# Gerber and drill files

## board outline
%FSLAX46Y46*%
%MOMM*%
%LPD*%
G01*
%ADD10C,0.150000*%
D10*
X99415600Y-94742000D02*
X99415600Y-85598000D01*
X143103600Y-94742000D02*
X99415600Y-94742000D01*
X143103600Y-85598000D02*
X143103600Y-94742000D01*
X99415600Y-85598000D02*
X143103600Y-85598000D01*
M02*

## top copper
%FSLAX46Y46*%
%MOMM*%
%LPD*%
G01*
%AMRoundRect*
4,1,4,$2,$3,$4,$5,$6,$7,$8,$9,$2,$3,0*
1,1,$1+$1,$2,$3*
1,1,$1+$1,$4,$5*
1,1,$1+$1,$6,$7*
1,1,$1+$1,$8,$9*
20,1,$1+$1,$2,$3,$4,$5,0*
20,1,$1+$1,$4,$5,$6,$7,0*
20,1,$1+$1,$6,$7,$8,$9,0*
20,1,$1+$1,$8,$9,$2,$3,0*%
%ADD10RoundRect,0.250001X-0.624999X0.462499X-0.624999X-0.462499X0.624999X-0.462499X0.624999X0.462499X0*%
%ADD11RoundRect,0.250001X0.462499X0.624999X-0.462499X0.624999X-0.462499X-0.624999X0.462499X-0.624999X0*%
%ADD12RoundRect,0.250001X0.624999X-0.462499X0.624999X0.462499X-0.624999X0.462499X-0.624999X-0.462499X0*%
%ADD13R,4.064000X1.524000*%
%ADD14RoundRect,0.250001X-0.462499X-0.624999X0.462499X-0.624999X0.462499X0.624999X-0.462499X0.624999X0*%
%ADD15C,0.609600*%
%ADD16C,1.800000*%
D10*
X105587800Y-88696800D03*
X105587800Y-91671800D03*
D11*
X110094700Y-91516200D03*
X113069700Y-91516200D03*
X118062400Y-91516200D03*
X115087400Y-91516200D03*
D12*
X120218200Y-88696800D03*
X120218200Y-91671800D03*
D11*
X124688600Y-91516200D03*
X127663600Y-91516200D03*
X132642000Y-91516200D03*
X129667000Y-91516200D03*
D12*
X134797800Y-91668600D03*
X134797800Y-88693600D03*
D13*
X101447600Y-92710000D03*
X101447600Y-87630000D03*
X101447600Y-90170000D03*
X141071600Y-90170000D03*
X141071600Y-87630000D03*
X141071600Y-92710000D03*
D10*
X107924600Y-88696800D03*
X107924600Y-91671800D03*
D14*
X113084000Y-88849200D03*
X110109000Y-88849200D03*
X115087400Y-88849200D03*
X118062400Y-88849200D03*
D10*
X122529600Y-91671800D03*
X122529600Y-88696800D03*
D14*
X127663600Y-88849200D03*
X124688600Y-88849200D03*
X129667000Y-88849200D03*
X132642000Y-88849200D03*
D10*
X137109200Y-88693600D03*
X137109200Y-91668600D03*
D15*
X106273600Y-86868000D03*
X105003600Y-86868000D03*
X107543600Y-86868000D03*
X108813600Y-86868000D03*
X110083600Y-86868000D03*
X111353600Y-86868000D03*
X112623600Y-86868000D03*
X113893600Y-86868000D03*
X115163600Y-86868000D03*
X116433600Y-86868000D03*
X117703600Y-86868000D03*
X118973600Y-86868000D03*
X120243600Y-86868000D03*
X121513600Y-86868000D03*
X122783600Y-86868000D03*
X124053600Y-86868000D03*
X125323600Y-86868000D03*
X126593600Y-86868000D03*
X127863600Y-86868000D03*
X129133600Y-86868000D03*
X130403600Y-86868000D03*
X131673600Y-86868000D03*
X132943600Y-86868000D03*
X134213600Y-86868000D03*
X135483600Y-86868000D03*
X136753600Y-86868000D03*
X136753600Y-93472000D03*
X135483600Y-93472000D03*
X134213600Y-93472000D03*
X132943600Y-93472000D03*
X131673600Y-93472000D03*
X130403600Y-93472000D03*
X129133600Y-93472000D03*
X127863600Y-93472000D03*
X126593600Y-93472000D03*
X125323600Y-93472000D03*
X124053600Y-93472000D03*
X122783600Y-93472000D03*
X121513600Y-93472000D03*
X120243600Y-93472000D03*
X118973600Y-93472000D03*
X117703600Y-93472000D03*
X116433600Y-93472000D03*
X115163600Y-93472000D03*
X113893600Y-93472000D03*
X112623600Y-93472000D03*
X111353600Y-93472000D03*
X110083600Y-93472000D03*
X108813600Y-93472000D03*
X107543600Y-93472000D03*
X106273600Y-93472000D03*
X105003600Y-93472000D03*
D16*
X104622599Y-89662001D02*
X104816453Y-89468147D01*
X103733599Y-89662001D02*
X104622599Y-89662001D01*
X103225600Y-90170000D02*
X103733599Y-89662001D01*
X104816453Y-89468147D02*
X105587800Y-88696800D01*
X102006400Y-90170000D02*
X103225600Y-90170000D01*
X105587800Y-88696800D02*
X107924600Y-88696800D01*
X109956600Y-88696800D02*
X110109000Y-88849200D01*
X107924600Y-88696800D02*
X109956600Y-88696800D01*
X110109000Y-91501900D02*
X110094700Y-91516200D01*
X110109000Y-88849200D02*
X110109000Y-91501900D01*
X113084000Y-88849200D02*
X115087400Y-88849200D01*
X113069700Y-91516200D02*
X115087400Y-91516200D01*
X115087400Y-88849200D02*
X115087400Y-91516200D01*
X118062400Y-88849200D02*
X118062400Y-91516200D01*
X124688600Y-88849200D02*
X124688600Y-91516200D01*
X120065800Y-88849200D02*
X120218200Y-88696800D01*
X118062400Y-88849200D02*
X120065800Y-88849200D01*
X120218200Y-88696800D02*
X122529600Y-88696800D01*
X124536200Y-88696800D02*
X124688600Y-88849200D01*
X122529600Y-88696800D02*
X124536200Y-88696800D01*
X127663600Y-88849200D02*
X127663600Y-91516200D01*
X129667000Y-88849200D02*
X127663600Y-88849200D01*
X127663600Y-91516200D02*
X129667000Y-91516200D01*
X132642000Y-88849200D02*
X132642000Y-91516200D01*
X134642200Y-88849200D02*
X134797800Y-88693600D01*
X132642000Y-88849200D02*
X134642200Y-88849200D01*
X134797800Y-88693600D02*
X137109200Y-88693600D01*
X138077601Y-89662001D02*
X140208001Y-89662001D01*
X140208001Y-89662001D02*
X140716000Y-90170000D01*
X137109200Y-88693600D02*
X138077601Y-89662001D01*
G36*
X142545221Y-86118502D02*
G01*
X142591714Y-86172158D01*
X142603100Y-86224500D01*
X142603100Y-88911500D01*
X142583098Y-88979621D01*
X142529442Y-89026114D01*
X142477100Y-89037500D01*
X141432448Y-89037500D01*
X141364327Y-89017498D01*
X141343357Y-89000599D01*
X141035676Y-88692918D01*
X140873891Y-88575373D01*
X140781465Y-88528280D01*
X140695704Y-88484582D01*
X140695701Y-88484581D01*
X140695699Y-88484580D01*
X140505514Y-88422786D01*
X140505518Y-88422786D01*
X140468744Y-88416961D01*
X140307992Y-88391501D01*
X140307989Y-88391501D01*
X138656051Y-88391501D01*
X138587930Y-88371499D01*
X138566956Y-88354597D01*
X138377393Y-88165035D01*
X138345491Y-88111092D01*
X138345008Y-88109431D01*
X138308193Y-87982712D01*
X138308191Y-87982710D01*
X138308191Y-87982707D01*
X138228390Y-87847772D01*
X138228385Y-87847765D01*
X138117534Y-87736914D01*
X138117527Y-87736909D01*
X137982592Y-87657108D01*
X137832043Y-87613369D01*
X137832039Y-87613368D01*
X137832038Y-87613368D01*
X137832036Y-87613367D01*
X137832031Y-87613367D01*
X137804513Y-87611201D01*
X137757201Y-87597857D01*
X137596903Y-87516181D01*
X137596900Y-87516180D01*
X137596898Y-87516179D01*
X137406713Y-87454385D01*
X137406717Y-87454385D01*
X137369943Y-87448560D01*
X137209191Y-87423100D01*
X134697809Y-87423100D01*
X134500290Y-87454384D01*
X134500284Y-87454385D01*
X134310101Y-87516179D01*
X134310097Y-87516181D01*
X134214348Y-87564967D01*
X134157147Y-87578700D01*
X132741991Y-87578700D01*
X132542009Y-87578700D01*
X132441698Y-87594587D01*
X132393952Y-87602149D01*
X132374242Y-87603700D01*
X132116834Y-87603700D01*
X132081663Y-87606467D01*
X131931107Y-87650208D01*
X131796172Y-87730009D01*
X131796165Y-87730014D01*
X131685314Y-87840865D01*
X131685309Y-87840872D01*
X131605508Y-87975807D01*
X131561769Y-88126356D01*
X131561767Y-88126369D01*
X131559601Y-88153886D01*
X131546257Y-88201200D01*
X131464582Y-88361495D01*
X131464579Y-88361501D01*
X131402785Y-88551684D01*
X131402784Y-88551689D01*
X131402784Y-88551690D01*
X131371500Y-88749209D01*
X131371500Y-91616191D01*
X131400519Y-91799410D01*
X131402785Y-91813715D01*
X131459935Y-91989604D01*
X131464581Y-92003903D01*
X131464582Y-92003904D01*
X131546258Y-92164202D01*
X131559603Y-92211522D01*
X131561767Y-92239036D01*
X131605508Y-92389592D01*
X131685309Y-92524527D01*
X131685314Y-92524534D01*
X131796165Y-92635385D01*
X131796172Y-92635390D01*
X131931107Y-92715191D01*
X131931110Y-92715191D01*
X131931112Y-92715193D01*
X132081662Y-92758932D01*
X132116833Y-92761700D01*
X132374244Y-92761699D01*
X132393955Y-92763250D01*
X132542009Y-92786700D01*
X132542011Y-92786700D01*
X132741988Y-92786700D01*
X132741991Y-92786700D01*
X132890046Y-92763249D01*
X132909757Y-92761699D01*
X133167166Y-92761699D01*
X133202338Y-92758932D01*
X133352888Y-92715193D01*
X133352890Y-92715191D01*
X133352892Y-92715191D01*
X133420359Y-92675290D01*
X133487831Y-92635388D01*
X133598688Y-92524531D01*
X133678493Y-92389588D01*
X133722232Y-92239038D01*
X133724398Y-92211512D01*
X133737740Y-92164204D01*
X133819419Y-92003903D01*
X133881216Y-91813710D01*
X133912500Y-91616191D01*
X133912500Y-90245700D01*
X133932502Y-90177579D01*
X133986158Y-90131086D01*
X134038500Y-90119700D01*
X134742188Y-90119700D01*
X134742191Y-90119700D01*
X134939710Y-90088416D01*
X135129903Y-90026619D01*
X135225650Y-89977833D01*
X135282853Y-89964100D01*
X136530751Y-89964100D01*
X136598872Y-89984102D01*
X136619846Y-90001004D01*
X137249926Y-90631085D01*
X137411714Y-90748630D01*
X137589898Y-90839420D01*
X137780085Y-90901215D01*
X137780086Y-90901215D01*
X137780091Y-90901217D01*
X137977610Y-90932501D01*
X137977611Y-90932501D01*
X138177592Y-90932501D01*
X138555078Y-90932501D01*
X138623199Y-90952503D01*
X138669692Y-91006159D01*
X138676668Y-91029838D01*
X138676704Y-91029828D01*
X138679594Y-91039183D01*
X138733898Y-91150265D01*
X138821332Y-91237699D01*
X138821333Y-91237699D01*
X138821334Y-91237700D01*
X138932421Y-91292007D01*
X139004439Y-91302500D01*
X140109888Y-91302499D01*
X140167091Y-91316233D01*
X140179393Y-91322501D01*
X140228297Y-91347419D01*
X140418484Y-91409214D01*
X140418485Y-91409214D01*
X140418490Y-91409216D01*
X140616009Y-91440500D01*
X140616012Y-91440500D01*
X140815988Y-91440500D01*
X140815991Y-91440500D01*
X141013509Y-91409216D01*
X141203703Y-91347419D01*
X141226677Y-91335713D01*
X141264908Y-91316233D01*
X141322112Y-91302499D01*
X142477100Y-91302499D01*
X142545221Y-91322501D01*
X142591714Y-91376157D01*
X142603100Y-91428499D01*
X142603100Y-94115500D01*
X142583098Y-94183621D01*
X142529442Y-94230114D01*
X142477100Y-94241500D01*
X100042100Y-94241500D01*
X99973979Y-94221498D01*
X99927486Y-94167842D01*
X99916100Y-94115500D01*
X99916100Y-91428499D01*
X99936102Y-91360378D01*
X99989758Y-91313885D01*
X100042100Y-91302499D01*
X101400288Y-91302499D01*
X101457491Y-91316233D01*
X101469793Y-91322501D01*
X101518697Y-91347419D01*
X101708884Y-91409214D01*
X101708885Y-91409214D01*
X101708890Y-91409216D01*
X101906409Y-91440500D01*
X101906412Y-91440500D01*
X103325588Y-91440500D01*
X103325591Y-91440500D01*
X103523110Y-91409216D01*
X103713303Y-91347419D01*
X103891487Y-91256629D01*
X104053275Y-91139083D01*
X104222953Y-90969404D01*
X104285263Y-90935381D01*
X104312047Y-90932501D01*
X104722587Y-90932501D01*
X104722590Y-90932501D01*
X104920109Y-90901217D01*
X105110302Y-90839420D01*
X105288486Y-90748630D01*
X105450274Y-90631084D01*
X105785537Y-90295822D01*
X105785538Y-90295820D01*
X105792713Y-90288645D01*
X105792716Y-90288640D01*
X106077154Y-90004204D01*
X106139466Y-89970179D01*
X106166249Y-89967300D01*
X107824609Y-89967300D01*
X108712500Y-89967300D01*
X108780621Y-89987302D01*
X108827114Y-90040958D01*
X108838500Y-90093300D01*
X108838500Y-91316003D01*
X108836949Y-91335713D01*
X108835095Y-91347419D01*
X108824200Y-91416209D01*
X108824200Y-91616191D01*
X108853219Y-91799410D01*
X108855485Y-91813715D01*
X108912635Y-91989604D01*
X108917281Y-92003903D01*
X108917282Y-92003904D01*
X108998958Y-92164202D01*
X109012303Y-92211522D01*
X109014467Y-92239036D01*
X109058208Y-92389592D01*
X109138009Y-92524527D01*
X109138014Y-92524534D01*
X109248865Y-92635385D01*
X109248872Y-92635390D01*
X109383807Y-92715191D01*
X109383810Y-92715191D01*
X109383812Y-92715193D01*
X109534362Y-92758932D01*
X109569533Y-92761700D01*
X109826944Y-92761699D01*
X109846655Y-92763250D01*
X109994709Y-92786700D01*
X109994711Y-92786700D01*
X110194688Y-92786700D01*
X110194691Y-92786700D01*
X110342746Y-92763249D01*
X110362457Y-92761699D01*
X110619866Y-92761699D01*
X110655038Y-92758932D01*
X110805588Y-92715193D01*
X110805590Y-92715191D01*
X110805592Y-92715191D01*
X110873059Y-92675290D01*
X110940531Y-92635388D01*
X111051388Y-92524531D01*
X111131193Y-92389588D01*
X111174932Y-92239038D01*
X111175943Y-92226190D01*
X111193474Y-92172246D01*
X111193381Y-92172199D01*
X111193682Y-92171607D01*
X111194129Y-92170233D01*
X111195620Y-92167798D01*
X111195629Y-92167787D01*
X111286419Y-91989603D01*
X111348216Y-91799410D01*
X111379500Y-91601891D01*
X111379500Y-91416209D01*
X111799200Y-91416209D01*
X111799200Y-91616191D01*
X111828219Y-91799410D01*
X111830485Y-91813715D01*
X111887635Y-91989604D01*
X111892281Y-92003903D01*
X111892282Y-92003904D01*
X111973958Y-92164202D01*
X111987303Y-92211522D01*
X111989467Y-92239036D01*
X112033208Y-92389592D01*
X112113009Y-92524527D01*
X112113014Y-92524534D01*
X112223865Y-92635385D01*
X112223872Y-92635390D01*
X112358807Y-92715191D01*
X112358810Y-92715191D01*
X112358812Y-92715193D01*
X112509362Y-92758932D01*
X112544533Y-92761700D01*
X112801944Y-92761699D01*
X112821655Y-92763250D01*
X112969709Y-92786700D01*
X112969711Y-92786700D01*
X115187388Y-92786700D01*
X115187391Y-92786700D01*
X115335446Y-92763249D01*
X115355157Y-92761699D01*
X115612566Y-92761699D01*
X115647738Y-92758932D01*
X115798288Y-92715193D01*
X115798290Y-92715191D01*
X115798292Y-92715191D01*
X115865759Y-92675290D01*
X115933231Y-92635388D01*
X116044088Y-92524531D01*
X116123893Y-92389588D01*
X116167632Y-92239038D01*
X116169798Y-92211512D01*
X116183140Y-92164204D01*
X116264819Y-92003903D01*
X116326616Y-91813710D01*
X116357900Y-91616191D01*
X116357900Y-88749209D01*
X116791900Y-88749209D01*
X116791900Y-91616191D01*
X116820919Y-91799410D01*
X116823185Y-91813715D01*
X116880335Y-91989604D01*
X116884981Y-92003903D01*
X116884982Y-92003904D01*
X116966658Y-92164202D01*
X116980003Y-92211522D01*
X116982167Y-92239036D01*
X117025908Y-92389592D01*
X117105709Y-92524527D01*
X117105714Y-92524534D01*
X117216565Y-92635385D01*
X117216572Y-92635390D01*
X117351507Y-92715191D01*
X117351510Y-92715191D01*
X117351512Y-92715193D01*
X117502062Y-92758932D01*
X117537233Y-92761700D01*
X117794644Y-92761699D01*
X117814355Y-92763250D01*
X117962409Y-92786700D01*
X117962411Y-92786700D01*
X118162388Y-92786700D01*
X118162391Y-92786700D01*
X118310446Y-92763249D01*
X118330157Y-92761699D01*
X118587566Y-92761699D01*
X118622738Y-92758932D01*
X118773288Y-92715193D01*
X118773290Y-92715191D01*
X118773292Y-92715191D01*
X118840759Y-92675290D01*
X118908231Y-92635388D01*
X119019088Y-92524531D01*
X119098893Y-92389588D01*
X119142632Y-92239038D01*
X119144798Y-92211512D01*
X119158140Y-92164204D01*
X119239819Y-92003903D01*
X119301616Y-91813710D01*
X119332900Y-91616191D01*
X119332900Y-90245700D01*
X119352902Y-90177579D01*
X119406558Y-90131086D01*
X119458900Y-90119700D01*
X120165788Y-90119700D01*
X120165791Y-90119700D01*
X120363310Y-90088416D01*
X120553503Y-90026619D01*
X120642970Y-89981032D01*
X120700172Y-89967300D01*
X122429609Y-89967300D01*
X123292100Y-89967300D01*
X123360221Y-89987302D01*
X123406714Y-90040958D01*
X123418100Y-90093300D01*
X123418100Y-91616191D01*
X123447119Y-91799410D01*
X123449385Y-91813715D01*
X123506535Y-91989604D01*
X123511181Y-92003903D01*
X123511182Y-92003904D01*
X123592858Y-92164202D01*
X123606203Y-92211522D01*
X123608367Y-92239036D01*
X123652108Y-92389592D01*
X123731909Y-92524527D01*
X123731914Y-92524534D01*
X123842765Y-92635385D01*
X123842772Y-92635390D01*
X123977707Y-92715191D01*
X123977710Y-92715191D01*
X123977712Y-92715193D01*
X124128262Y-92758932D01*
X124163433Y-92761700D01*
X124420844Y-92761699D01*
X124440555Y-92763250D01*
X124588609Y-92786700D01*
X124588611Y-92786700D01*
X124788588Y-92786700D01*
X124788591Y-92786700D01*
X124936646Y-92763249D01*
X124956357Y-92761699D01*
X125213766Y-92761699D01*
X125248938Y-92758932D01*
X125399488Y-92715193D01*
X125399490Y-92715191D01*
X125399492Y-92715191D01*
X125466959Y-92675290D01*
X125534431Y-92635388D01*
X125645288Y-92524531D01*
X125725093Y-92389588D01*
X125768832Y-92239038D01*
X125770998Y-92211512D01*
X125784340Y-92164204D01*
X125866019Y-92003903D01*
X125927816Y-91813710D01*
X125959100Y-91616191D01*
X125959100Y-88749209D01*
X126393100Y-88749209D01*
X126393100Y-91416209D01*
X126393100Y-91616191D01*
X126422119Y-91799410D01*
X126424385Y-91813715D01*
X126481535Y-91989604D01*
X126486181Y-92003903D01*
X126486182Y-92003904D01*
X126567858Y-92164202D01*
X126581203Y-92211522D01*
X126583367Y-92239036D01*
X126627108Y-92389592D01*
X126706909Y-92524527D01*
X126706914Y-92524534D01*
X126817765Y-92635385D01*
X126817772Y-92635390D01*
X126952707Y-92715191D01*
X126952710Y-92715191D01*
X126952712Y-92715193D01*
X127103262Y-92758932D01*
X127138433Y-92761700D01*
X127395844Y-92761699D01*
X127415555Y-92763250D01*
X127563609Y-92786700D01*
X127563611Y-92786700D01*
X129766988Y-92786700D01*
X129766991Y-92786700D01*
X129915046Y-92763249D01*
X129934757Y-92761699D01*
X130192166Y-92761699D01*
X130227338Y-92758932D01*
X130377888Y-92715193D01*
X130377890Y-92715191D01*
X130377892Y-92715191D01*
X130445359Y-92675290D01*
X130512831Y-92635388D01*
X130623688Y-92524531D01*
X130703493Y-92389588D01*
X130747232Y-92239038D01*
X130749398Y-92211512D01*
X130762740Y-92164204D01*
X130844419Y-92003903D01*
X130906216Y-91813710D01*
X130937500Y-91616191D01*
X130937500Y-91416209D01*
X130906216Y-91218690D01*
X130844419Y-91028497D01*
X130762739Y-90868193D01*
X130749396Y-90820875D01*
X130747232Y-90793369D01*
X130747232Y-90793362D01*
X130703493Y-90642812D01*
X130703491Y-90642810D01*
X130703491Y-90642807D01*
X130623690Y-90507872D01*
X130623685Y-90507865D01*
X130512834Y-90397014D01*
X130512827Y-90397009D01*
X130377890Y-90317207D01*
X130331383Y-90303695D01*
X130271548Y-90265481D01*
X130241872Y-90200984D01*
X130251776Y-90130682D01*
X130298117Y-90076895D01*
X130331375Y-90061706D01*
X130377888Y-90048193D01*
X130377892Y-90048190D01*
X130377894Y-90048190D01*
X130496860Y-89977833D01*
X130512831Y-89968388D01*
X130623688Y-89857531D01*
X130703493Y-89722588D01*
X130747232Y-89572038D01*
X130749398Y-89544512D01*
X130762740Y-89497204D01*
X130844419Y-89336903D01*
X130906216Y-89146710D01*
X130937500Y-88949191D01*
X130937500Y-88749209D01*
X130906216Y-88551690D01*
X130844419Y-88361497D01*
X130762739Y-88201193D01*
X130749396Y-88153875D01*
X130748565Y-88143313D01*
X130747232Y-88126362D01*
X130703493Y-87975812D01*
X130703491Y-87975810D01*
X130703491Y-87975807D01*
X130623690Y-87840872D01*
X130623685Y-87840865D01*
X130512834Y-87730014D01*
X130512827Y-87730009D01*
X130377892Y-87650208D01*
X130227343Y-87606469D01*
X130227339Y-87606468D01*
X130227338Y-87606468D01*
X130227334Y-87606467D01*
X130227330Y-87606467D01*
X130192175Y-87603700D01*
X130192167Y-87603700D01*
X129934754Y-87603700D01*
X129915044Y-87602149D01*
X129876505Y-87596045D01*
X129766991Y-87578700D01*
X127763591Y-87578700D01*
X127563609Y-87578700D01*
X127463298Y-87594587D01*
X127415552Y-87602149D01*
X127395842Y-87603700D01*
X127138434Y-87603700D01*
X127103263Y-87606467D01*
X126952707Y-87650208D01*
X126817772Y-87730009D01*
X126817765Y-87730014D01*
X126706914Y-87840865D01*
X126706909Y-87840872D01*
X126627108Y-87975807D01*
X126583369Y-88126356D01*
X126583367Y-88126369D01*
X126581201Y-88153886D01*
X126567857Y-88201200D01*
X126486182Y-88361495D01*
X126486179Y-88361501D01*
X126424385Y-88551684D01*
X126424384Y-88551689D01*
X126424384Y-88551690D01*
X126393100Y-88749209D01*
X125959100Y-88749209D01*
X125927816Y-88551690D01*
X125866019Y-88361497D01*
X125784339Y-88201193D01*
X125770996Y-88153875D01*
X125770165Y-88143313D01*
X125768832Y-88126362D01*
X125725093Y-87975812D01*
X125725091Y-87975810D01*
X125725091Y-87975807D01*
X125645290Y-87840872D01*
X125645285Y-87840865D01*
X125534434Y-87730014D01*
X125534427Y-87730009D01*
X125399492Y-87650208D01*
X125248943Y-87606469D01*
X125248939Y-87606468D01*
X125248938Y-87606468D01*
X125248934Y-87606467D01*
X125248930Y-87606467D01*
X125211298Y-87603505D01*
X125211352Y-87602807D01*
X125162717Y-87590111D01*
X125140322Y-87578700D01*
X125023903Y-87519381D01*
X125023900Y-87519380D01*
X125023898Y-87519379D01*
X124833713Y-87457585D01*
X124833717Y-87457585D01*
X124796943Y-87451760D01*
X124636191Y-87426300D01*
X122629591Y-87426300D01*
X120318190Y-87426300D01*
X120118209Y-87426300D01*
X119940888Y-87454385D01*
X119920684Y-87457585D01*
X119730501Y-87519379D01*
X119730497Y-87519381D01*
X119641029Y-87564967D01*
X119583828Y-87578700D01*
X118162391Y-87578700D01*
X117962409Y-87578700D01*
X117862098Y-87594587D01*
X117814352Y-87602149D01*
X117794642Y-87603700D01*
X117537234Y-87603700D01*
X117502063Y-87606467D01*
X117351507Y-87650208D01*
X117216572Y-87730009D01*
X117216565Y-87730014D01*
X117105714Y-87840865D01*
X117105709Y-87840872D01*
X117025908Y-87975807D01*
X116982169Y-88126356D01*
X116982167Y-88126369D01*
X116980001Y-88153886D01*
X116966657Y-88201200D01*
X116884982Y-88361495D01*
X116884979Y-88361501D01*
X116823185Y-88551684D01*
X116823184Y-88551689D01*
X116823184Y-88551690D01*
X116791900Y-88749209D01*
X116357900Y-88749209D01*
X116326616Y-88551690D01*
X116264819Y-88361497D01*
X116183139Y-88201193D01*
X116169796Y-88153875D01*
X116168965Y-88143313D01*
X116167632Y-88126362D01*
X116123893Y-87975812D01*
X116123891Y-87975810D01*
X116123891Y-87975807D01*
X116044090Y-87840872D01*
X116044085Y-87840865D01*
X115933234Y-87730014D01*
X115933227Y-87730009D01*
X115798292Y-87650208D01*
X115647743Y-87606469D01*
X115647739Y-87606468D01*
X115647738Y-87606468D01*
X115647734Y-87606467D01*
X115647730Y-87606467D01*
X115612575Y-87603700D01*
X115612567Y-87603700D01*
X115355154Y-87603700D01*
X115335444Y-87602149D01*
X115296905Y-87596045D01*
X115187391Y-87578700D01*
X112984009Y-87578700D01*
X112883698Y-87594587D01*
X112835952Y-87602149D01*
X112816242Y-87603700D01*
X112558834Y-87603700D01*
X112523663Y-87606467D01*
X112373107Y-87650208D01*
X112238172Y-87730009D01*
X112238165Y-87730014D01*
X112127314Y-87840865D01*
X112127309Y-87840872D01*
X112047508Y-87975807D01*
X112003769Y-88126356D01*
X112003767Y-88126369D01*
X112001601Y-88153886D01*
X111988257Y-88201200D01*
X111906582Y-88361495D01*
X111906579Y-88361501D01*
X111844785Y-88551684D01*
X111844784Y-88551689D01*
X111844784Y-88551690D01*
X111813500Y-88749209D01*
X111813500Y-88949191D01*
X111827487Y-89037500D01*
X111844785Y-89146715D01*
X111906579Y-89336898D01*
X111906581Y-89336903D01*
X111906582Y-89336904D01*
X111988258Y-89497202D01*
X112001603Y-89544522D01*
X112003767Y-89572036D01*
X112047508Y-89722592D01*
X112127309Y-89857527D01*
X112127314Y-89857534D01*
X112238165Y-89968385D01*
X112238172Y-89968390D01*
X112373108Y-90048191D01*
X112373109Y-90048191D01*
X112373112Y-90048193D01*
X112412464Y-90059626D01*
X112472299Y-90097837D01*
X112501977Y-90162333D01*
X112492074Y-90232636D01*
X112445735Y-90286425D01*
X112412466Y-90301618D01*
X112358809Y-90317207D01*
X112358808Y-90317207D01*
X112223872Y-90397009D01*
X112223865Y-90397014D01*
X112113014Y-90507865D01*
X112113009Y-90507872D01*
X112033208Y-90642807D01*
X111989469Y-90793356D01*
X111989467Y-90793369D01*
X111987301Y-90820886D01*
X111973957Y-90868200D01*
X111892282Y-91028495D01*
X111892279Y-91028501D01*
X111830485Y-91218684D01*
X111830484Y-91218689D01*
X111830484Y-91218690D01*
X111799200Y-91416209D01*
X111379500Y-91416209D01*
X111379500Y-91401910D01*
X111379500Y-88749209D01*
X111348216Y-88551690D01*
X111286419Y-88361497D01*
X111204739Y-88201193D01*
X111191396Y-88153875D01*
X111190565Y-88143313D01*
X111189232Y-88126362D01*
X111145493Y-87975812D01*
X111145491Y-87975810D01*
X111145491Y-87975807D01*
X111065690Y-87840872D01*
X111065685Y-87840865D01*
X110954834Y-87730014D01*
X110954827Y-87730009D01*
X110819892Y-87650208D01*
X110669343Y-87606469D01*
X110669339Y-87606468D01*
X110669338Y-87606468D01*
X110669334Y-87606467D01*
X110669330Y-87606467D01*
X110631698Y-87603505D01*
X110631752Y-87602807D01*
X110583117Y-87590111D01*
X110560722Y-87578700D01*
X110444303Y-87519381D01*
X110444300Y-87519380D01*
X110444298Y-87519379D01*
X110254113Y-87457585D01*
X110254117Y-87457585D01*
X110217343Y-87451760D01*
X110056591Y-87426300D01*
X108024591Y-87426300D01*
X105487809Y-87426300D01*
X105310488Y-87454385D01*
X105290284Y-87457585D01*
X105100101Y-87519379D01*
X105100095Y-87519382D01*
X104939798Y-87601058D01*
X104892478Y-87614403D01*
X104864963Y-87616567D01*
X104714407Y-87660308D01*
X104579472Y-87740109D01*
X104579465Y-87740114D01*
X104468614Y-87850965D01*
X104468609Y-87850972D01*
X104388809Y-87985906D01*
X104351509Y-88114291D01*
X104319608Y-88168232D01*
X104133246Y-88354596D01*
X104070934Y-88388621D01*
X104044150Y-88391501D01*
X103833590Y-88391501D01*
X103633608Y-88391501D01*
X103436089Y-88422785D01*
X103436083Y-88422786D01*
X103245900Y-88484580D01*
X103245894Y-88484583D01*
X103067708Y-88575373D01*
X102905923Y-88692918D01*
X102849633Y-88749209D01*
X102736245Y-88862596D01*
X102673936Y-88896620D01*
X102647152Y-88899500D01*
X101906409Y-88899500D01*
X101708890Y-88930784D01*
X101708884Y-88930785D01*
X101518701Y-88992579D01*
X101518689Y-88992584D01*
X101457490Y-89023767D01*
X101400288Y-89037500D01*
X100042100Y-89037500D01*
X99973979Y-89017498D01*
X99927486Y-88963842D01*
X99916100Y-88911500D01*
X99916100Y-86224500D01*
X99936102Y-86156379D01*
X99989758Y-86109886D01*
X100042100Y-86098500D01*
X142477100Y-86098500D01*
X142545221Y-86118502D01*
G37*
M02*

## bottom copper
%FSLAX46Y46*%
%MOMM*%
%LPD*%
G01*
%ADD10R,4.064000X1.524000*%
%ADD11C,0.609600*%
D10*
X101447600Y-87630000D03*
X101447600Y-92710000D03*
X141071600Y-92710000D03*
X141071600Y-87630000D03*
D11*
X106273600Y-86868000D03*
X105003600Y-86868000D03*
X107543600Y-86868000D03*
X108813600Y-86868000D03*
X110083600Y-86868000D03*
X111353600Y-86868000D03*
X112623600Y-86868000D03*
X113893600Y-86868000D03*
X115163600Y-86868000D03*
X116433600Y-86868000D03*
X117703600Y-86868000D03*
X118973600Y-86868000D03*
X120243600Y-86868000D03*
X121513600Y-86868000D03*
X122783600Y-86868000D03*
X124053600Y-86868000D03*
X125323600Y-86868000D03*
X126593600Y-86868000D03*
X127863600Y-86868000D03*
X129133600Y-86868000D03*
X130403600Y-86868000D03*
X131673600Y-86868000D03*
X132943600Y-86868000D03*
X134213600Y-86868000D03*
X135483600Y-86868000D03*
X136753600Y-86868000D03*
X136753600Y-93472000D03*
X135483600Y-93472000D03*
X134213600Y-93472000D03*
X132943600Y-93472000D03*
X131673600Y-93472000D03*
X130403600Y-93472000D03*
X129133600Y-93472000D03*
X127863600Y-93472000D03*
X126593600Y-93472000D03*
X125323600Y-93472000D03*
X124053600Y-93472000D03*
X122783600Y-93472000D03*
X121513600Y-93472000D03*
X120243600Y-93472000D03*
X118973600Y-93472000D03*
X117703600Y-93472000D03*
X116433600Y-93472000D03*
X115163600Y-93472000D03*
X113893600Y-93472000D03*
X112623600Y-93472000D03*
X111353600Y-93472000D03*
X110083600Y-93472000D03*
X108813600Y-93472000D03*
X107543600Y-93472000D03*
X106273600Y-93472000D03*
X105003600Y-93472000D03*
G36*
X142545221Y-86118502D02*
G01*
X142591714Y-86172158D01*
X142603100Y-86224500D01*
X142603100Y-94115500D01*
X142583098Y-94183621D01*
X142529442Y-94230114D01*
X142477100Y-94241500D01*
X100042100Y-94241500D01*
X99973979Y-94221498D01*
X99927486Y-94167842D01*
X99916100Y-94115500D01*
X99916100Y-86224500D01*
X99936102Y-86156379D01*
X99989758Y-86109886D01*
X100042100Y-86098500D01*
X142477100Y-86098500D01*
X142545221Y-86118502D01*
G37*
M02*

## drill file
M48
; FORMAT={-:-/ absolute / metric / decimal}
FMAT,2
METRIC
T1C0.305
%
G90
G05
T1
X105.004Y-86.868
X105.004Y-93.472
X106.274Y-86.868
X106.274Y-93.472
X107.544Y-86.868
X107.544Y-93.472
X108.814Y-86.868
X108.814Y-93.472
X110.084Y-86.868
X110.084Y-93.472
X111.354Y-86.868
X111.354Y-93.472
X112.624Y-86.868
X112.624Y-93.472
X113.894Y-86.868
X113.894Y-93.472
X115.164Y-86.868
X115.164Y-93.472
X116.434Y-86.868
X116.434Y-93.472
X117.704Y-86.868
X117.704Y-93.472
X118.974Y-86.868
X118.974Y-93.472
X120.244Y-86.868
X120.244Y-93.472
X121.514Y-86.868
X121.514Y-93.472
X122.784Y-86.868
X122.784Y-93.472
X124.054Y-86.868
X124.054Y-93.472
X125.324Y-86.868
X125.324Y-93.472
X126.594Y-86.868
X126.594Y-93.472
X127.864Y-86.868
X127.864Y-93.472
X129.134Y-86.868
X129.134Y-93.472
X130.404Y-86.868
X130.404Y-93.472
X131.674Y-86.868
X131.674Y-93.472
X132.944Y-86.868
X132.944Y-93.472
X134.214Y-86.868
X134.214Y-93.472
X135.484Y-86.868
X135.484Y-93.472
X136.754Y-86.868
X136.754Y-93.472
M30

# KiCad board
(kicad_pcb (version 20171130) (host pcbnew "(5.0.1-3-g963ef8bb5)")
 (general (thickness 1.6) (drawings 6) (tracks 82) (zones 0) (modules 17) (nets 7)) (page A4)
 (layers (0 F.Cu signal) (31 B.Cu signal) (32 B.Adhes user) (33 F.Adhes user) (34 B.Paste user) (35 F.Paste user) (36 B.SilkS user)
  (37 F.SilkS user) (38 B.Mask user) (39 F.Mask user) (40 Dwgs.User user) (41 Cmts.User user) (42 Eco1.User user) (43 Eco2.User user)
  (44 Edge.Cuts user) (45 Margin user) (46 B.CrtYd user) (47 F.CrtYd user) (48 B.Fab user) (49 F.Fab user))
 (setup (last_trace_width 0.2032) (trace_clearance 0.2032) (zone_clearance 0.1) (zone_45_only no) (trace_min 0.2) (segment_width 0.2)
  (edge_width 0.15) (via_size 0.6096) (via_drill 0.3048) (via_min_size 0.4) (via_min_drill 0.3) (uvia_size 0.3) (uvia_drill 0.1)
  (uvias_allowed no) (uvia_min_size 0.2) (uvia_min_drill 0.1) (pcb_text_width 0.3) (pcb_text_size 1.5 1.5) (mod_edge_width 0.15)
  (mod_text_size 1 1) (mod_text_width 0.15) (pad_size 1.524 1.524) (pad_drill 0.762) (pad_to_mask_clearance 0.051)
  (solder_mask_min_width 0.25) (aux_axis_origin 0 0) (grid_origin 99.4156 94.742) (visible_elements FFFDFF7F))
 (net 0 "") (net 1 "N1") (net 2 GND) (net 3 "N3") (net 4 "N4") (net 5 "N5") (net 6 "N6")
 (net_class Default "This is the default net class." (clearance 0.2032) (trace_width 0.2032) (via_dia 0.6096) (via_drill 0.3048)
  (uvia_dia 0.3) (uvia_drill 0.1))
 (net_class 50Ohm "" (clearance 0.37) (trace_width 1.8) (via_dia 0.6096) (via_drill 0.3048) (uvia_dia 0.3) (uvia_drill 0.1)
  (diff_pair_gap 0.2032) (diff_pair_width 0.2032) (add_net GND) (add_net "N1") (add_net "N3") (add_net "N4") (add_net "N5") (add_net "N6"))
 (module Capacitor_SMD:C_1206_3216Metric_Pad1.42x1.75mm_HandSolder (layer F.Cu) (at 105.5878 90.1843 270)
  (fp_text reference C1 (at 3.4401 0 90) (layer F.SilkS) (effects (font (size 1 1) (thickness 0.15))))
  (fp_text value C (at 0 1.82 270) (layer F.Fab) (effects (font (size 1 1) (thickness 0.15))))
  (pad 1 smd roundrect (at -1.4875 0 270) (size 1.425 1.75) (layers F.Cu F.Paste F.Mask) (roundrect_rratio 0.175439) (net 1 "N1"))
  (pad 2 smd roundrect (at 1.4875 0 270) (size 1.425 1.75) (layers F.Cu F.Paste F.Mask) (roundrect_rratio 0.175439) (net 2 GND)))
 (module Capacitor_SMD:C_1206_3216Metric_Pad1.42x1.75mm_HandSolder (layer F.Cu) (at 111.5822 91.5162 180)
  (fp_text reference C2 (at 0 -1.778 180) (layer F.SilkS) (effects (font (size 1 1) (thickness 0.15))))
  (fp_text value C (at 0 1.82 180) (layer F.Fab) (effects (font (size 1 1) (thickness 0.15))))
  (pad 2 smd roundrect (at 1.4875 0 180) (size 1.425 1.75) (layers F.Cu F.Paste F.Mask) (roundrect_rratio 0.175439) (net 1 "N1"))
  (pad 1 smd roundrect (at -1.4875 0 180) (size 1.425 1.75) (layers F.Cu F.Paste F.Mask) (roundrect_rratio 0.175439) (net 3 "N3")))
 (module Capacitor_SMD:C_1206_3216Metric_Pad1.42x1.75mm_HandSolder (layer F.Cu) (at 116.5749 91.5162 180)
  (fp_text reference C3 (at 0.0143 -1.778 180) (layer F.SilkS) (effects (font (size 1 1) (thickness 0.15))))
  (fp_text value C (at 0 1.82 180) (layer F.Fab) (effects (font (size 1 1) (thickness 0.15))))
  (pad 1 smd roundrect (at -1.4875 0 180) (size 1.425 1.75) (layers F.Cu F.Paste F.Mask) (roundrect_rratio 0.175439) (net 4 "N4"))
  (pad 2 smd roundrect (at 1.4875 0 180) (size 1.425 1.75) (layers F.Cu F.Paste F.Mask) (roundrect_rratio 0.175439) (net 3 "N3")))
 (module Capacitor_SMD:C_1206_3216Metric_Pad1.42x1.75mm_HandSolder (layer F.Cu) (at 120.2182 90.1843 90)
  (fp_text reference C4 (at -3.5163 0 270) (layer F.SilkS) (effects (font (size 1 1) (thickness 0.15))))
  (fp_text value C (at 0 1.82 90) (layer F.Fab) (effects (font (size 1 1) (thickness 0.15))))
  (pad 2 smd roundrect (at 1.4875 0 90) (size 1.425 1.75) (layers F.Cu F.Paste F.Mask) (roundrect_rratio 0.175439) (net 4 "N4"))
  (pad 1 smd roundrect (at -1.4875 0 90) (size 1.425 1.75) (layers F.Cu F.Paste F.Mask) (roundrect_rratio 0.175439) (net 2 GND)))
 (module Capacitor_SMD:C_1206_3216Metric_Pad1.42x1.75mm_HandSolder (layer F.Cu) (at 126.1761 91.5162 180)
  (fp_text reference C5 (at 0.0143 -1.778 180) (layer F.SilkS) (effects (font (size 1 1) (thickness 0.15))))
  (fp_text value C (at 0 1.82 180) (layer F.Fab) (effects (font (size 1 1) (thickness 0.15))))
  (pad 2 smd roundrect (at 1.4875 0 180) (size 1.425 1.75) (layers F.Cu F.Paste F.Mask) (roundrect_rratio 0.175439) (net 4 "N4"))
  (pad 1 smd roundrect (at -1.4875 0 180) (size 1.425 1.75) (layers F.Cu F.Paste F.Mask) (roundrect_rratio 0.175439) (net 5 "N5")))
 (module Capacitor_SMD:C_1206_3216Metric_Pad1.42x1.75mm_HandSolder (layer F.Cu) (at 131.1545 91.5162 180)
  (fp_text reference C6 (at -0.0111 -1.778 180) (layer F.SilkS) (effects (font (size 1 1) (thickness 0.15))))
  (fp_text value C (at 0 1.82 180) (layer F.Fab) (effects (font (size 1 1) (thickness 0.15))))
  (pad 1 smd roundrect (at -1.4875 0 180) (size 1.425 1.75) (layers F.Cu F.Paste F.Mask) (roundrect_rratio 0.175439) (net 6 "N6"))
  (pad 2 smd roundrect (at 1.4875 0 180) (size 1.425 1.75) (layers F.Cu F.Paste F.Mask) (roundrect_rratio 0.175439) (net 5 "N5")))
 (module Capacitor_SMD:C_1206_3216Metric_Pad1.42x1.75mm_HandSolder (layer F.Cu) (at 134.7978 90.1811 90)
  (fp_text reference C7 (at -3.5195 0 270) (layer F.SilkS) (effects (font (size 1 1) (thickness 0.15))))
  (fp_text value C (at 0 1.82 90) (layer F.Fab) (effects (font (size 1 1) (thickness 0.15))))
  (pad 1 smd roundrect (at -1.4875 0 90) (size 1.425 1.75) (layers F.Cu F.Paste F.Mask) (roundrect_rratio 0.175439) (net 2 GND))
  (pad 2 smd roundrect (at 1.4875 0 90) (size 1.425 1.75) (layers F.Cu F.Paste F.Mask) (roundrect_rratio 0.175439) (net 6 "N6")))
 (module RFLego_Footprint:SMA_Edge (layer F.Cu) (at 99.4156 90.17)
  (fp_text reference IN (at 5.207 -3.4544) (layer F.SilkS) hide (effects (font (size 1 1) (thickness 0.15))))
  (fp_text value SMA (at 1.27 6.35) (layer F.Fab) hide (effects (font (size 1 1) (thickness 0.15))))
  (pad 2 smd rect (at 2.032 2.54) (size 4.064 1.524) (layers F.Cu F.Mask) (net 2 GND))
  (pad 2 smd rect (at 2.032 -2.54) (size 4.064 1.524) (layers B.Cu B.Mask) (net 2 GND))
  (pad 2 smd rect (at 2.032 2.54) (size 4.064 1.524) (layers B.Cu B.Mask) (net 2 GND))
  (pad 2 smd rect (at 2.032 -2.54) (size 4.064 1.524) (layers F.Cu F.Mask) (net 2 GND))
  (pad 1 smd rect (at 2.032 0) (size 4.064 1.524) (layers F.Cu F.Mask) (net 1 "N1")))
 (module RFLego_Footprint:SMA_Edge (layer F.Cu) (at 139.0396 90.17)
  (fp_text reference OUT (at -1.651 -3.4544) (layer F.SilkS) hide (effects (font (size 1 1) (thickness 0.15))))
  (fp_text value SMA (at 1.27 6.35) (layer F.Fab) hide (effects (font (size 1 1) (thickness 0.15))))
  (pad 1 smd rect (at 2.032 0) (size 4.064 1.524) (layers F.Cu F.Mask) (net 6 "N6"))
  (pad 2 smd rect (at 2.032 -2.54) (size 4.064 1.524) (layers F.Cu F.Mask) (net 2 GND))
  (pad 2 smd rect (at 2.032 2.54) (size 4.064 1.524) (layers B.Cu B.Mask) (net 2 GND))
  (pad 2 smd rect (at 2.032 -2.54) (size 4.064 1.524) (layers B.Cu B.Mask) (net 2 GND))
  (pad 2 smd rect (at 2.032 2.54) (size 4.064 1.524) (layers F.Cu F.Mask) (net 2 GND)))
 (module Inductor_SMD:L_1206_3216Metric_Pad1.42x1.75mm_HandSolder (layer F.Cu) (at 107.9246 90.1843 270)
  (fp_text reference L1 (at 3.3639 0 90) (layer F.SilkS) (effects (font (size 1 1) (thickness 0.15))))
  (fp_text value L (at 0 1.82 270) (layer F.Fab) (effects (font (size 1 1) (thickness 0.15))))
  (pad 1 smd roundrect (at -1.4875 0 270) (size 1.425 1.75) (layers F.Cu F.Paste F.Mask) (roundrect_rratio 0.175439) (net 1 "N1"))
  (pad 2 smd roundrect (at 1.4875 0 270) (size 1.425 1.75) (layers F.Cu F.Paste F.Mask) (roundrect_rratio 0.175439) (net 2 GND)))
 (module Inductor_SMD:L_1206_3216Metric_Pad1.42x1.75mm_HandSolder (layer F.Cu) (at 111.5965 88.8492)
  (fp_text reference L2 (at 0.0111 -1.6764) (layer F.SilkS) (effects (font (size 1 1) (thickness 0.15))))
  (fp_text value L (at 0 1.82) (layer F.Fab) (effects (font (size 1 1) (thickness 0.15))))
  (pad 2 smd roundrect (at 1.4875 0) (size 1.425 1.75) (layers F.Cu F.Paste F.Mask) (roundrect_rratio 0.175439) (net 3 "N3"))
  (pad 1 smd roundrect (at -1.4875 0) (size 1.425 1.75) (layers F.Cu F.Paste F.Mask) (roundrect_rratio 0.175439) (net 1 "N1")))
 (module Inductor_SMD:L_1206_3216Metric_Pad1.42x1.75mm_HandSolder (layer F.Cu) (at 116.5749 88.8492)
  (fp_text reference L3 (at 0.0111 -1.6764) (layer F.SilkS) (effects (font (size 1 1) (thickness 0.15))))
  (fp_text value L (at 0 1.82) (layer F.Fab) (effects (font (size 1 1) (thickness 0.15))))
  (pad 1 smd roundrect (at -1.4875 0) (size 1.425 1.75) (layers F.Cu F.Paste F.Mask) (roundrect_rratio 0.175439) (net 3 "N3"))
  (pad 2 smd roundrect (at 1.4875 0) (size 1.425 1.75) (layers F.Cu F.Paste F.Mask) (roundrect_rratio 0.175439) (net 4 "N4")))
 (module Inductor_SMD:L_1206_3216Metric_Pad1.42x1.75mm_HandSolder (layer F.Cu) (at 122.5296 90.1843 270)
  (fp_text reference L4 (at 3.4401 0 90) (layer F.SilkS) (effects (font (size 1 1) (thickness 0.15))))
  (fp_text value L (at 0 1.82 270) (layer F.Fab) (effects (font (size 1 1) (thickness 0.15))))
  (pad 2 smd roundrect (at 1.4875 0 270) (size 1.425 1.75) (layers F.Cu F.Paste F.Mask) (roundrect_rratio 0.175439) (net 2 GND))
  (pad 1 smd roundrect (at -1.4875 0 270) (size 1.425 1.75) (layers F.Cu F.Paste F.Mask) (roundrect_rratio 0.175439) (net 4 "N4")))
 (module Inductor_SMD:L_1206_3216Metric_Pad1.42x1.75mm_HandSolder (layer F.Cu) (at 126.1761 88.8492)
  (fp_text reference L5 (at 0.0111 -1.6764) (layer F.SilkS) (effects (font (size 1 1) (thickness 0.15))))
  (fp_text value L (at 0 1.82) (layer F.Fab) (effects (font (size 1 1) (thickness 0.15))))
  (pad 2 smd roundrect (at 1.4875 0) (size 1.425 1.75) (layers F.Cu F.Paste F.Mask) (roundrect_rratio 0.175439) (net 5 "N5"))
  (pad 1 smd roundrect (at -1.4875 0) (size 1.425 1.75) (layers F.Cu F.Paste F.Mask) (roundrect_rratio 0.175439) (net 4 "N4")))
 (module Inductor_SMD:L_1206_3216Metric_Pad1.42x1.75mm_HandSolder (layer F.Cu) (at 131.1545 88.8492)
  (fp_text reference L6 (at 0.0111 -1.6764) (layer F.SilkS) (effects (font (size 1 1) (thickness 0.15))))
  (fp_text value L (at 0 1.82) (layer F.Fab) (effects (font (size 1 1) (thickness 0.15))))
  (pad 1 smd roundrect (at -1.4875 0) (size 1.425 1.75) (layers F.Cu F.Paste F.Mask) (roundrect_rratio 0.175439) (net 5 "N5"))
  (pad 2 smd roundrect (at 1.4875 0) (size 1.425 1.75) (layers F.Cu F.Paste F.Mask) (roundrect_rratio 0.175439) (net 6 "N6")))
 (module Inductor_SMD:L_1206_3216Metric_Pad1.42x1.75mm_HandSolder (layer F.Cu) (at 137.1092 90.1811 270)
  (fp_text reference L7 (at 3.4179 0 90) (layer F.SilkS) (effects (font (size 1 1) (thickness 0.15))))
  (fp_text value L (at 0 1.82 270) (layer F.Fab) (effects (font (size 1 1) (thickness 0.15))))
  (pad 1 smd roundrect (at -1.4875 0 270) (size 1.425 1.75) (layers F.Cu F.Paste F.Mask) (roundrect_rratio 0.175439) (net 6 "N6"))
  (pad 2 smd roundrect (at 1.4875 0 270) (size 1.425 1.75) (layers F.Cu F.Paste F.Mask) (roundrect_rratio 0.175439) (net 2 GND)))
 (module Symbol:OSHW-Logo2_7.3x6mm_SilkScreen (layer B.Cu) (at 107.1118 90.1446 180)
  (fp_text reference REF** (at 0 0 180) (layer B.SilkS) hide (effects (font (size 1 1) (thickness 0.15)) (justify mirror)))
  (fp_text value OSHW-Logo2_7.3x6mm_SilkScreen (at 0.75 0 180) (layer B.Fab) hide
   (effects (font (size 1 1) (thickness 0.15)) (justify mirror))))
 (gr_line (start 99.4156 94.742) (end 99.4156 85.598) (layer Edge.Cuts) (width 0.15))
 (gr_line (start 143.1036 94.742) (end 99.4156 94.742) (layer Edge.Cuts) (width 0.15))
 (gr_line (start 143.1036 85.598) (end 143.1036 94.742) (layer Edge.Cuts) (width 0.15))
 (gr_line (start 99.4156 85.598) (end 143.1036 85.598) (layer Edge.Cuts) (width 0.15))
 (segment (start 104.622599 89.662001) (end 104.816453 89.468147) (width 1.8) (layer F.Cu) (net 1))
 (segment (start 103.733599 89.662001) (end 104.622599 89.662001) (width 1.8) (layer F.Cu) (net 1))
 (segment (start 103.2256 90.17) (end 103.733599 89.662001) (width 1.8) (layer F.Cu) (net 1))
 (segment (start 104.816453 89.468147) (end 105.5878 88.6968) (width 1.8) (layer F.Cu) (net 1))
 (segment (start 102.0064 90.17) (end 103.2256 90.17) (width 1.8) (layer F.Cu) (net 1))
 (segment (start 105.5878 88.6968) (end 107.9246 88.6968) (width 1.8) (layer F.Cu) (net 1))
 (segment (start 109.9566 88.6968) (end 110.109 88.8492) (width 1.8) (layer F.Cu) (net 1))
 (segment (start 107.9246 88.6968) (end 109.9566 88.6968) (width 1.8) (layer F.Cu) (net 1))
 (segment (start 110.109 91.5019) (end 110.0947 91.5162) (width 1.8) (layer F.Cu) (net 1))
 (segment (start 110.109 88.8492) (end 110.109 91.5019) (width 1.8) (layer F.Cu) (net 1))
 (via (at 106.2736 86.868) (size 0.6096) (drill 0.3048) (layers F.Cu B.Cu) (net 2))
 (via (at 105.0036 86.868) (size 0.6096) (drill 0.3048) (layers F.Cu B.Cu) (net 2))
 (via (at 107.5436 86.868) (size 0.6096) (drill 0.3048) (layers F.Cu B.Cu) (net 2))
 (via (at 108.8136 86.868) (size 0.6096) (drill 0.3048) (layers F.Cu B.Cu) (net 2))
 (via (at 110.0836 86.868) (size 0.6096) (drill 0.3048) (layers F.Cu B.Cu) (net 2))
 (via (at 111.3536 86.868) (size 0.6096) (drill 0.3048) (layers F.Cu B.Cu) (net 2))
 (via (at 112.6236 86.868) (size 0.6096) (drill 0.3048) (layers F.Cu B.Cu) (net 2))
 (via (at 113.8936 86.868) (size 0.6096) (drill 0.3048) (layers F.Cu B.Cu) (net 2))
 (via (at 115.1636 86.868) (size 0.6096) (drill 0.3048) (layers F.Cu B.Cu) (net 2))
 (via (at 116.4336 86.868) (size 0.6096) (drill 0.3048) (layers F.Cu B.Cu) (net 2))
 (via (at 117.7036 86.868) (size 0.6096) (drill 0.3048) (layers F.Cu B.Cu) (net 2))
 (via (at 118.9736 86.868) (size 0.6096) (drill 0.3048) (layers F.Cu B.Cu) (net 2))
 (via (at 120.2436 86.868) (size 0.6096) (drill 0.3048) (layers F.Cu B.Cu) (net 2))
 (via (at 121.5136 86.868) (size 0.6096) (drill 0.3048) (layers F.Cu B.Cu) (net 2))
 (via (at 122.7836 86.868) (size 0.6096) (drill 0.3048) (layers F.Cu B.Cu) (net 2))
 (via (at 124.0536 86.868) (size 0.6096) (drill 0.3048) (layers F.Cu B.Cu) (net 2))
 (via (at 125.3236 86.868) (size 0.6096) (drill 0.3048) (layers F.Cu B.Cu) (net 2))
 (via (at 126.5936 86.868) (size 0.6096) (drill 0.3048) (layers F.Cu B.Cu) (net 2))
 (via (at 127.8636 86.868) (size 0.6096) (drill 0.3048) (layers F.Cu B.Cu) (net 2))
 (via (at 129.1336 86.868) (size 0.6096) (drill 0.3048) (layers F.Cu B.Cu) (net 2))
 (via (at 130.4036 86.868) (size 0.6096) (drill 0.3048) (layers F.Cu B.Cu) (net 2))
 (via (at 131.6736 86.868) (size 0.6096) (drill 0.3048) (layers F.Cu B.Cu) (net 2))
 (via (at 132.9436 86.868) (size 0.6096) (drill 0.3048) (layers F.Cu B.Cu) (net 2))
 (via (at 134.2136 86.868) (size 0.6096) (drill 0.3048) (layers F.Cu B.Cu) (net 2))
 (via (at 135.4836 86.868) (size 0.6096) (drill 0.3048) (layers F.Cu B.Cu) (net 2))
 (via (at 136.7536 86.868) (size 0.6096) (drill 0.3048) (layers F.Cu B.Cu) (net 2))
 (via (at 136.7536 93.472) (size 0.6096) (drill 0.3048) (layers F.Cu B.Cu) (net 2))
 (via (at 135.4836 93.472) (size 0.6096) (drill 0.3048) (layers F.Cu B.Cu) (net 2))
 (via (at 134.2136 93.472) (size 0.6096) (drill 0.3048) (layers F.Cu B.Cu) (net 2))
 (via (at 132.9436 93.472) (size 0.6096) (drill 0.3048) (layers F.Cu B.Cu) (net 2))
 (via (at 131.6736 93.472) (size 0.6096) (drill 0.3048) (layers F.Cu B.Cu) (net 2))
 (via (at 130.4036 93.472) (size 0.6096) (drill 0.3048) (layers F.Cu B.Cu) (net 2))
 (via (at 129.1336 93.472) (size 0.6096) (drill 0.3048) (layers F.Cu B.Cu) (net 2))
 (via (at 127.8636 93.472) (size 0.6096) (drill 0.3048) (layers F.Cu B.Cu) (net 2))
 (via (at 126.5936 93.472) (size 0.6096) (drill 0.3048) (layers F.Cu B.Cu) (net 2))
 (via (at 125.3236 93.472) (size 0.6096) (drill 0.3048) (layers F.Cu B.Cu) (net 2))
 (via (at 124.0536 93.472) (size 0.6096) (drill 0.3048) (layers F.Cu B.Cu) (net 2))
 (via (at 122.7836 93.472) (size 0.6096) (drill 0.3048) (layers F.Cu B.Cu) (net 2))
 (via (at 121.5136 93.472) (size 0.6096) (drill 0.3048) (layers F.Cu B.Cu) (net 2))
 (via (at 120.2436 93.472) (size 0.6096) (drill 0.3048) (layers F.Cu B.Cu) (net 2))
 (via (at 118.9736 93.472) (size 0.6096) (drill 0.3048) (layers F.Cu B.Cu) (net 2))
 (via (at 117.7036 93.472) (size 0.6096) (drill 0.3048) (layers F.Cu B.Cu) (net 2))
 (via (at 116.4336 93.472) (size 0.6096) (drill 0.3048) (layers F.Cu B.Cu) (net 2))
 (via (at 115.1636 93.472) (size 0.6096) (drill 0.3048) (layers F.Cu B.Cu) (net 2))
 (via (at 113.8936 93.472) (size 0.6096) (drill 0.3048) (layers F.Cu B.Cu) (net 2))
 (via (at 112.6236 93.472) (size 0.6096) (drill 0.3048) (layers F.Cu B.Cu) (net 2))
 (via (at 111.3536 93.472) (size 0.6096) (drill 0.3048) (layers F.Cu B.Cu) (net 2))
 (via (at 110.0836 93.472) (size 0.6096) (drill 0.3048) (layers F.Cu B.Cu) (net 2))
 (via (at 108.8136 93.472) (size 0.6096) (drill 0.3048) (layers F.Cu B.Cu) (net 2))
 (via (at 107.5436 93.472) (size 0.6096) (drill 0.3048) (layers F.Cu B.Cu) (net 2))
 (via (at 106.2736 93.472) (size 0.6096) (drill 0.3048) (layers F.Cu B.Cu) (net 2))
 (via (at 105.0036 93.472) (size 0.6096) (drill 0.3048) (layers F.Cu B.Cu) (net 2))
 (segment (start 113.084 88.8492) (end 115.0874 88.8492) (width 1.8) (layer F.Cu) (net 3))
 (segment (start 113.0697 91.5162) (end 115.0874 91.5162) (width 1.8) (layer F.Cu) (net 3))
 (segment (start 115.0874 88.8492) (end 115.0874 91.5162) (width 1.8) (layer F.Cu) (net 3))
 (segment (start 118.0624 88.8492) (end 118.0624 91.5162) (width 1.8) (layer F.Cu) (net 4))
 (segment (start 124.6886 88.8492) (end 124.6886 91.5162) (width 1.8) (layer F.Cu) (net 4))
 (segment (start 120.0658 88.8492) (end 120.2182 88.6968) (width 1.8) (layer F.Cu) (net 4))
 (segment (start 118.0624 88.8492) (end 120.0658 88.8492) (width 1.8) (layer F.Cu) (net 4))
 (segment (start 120.2182 88.6968) (end 122.5296 88.6968) (width 1.8) (layer F.Cu) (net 4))
 (segment (start 124.5362 88.6968) (end 124.6886 88.8492) (width 1.8) (layer F.Cu) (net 4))
 (segment (start 122.5296 88.6968) (end 124.5362 88.6968) (width 1.8) (layer F.Cu) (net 4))
 (segment (start 127.6636 88.8492) (end 127.6636 91.5162) (width 1.8) (layer F.Cu) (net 5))
 (segment (start 129.667 88.8492) (end 127.6636 88.8492) (width 1.8) (layer F.Cu) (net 5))
 (segment (start 127.6636 91.5162) (end 129.667 91.5162) (width 1.8) (layer F.Cu) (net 5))
 (segment (start 132.642 88.8492) (end 132.642 91.5162) (width 1.8) (layer F.Cu) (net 6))
 (segment (start 134.6422 88.8492) (end 134.7978 88.6936) (width 1.8) (layer F.Cu) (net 6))
 (segment (start 132.642 88.8492) (end 134.6422 88.8492) (width 1.8) (layer F.Cu) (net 6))
 (segment (start 134.7978 88.6936) (end 137.1092 88.6936) (width 1.8) (layer F.Cu) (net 6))
 (segment (start 138.077601 89.662001) (end 140.208001 89.662001) (width 1.8) (layer F.Cu) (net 6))
 (segment (start 140.208001 89.662001) (end 140.716 90.17) (width 1.8) (layer F.Cu) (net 6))
 (segment (start 137.1092 88.6936) (end 138.077601 89.662001) (width 1.8) (layer F.Cu) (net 6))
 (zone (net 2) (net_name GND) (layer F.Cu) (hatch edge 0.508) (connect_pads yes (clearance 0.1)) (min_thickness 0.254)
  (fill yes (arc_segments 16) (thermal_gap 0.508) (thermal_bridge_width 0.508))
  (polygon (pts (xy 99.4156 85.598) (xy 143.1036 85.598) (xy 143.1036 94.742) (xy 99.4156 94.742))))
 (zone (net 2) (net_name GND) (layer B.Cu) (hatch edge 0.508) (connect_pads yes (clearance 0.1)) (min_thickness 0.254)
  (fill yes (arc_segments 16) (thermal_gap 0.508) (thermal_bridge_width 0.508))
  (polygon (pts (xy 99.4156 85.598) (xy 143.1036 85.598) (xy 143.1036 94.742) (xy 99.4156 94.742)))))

